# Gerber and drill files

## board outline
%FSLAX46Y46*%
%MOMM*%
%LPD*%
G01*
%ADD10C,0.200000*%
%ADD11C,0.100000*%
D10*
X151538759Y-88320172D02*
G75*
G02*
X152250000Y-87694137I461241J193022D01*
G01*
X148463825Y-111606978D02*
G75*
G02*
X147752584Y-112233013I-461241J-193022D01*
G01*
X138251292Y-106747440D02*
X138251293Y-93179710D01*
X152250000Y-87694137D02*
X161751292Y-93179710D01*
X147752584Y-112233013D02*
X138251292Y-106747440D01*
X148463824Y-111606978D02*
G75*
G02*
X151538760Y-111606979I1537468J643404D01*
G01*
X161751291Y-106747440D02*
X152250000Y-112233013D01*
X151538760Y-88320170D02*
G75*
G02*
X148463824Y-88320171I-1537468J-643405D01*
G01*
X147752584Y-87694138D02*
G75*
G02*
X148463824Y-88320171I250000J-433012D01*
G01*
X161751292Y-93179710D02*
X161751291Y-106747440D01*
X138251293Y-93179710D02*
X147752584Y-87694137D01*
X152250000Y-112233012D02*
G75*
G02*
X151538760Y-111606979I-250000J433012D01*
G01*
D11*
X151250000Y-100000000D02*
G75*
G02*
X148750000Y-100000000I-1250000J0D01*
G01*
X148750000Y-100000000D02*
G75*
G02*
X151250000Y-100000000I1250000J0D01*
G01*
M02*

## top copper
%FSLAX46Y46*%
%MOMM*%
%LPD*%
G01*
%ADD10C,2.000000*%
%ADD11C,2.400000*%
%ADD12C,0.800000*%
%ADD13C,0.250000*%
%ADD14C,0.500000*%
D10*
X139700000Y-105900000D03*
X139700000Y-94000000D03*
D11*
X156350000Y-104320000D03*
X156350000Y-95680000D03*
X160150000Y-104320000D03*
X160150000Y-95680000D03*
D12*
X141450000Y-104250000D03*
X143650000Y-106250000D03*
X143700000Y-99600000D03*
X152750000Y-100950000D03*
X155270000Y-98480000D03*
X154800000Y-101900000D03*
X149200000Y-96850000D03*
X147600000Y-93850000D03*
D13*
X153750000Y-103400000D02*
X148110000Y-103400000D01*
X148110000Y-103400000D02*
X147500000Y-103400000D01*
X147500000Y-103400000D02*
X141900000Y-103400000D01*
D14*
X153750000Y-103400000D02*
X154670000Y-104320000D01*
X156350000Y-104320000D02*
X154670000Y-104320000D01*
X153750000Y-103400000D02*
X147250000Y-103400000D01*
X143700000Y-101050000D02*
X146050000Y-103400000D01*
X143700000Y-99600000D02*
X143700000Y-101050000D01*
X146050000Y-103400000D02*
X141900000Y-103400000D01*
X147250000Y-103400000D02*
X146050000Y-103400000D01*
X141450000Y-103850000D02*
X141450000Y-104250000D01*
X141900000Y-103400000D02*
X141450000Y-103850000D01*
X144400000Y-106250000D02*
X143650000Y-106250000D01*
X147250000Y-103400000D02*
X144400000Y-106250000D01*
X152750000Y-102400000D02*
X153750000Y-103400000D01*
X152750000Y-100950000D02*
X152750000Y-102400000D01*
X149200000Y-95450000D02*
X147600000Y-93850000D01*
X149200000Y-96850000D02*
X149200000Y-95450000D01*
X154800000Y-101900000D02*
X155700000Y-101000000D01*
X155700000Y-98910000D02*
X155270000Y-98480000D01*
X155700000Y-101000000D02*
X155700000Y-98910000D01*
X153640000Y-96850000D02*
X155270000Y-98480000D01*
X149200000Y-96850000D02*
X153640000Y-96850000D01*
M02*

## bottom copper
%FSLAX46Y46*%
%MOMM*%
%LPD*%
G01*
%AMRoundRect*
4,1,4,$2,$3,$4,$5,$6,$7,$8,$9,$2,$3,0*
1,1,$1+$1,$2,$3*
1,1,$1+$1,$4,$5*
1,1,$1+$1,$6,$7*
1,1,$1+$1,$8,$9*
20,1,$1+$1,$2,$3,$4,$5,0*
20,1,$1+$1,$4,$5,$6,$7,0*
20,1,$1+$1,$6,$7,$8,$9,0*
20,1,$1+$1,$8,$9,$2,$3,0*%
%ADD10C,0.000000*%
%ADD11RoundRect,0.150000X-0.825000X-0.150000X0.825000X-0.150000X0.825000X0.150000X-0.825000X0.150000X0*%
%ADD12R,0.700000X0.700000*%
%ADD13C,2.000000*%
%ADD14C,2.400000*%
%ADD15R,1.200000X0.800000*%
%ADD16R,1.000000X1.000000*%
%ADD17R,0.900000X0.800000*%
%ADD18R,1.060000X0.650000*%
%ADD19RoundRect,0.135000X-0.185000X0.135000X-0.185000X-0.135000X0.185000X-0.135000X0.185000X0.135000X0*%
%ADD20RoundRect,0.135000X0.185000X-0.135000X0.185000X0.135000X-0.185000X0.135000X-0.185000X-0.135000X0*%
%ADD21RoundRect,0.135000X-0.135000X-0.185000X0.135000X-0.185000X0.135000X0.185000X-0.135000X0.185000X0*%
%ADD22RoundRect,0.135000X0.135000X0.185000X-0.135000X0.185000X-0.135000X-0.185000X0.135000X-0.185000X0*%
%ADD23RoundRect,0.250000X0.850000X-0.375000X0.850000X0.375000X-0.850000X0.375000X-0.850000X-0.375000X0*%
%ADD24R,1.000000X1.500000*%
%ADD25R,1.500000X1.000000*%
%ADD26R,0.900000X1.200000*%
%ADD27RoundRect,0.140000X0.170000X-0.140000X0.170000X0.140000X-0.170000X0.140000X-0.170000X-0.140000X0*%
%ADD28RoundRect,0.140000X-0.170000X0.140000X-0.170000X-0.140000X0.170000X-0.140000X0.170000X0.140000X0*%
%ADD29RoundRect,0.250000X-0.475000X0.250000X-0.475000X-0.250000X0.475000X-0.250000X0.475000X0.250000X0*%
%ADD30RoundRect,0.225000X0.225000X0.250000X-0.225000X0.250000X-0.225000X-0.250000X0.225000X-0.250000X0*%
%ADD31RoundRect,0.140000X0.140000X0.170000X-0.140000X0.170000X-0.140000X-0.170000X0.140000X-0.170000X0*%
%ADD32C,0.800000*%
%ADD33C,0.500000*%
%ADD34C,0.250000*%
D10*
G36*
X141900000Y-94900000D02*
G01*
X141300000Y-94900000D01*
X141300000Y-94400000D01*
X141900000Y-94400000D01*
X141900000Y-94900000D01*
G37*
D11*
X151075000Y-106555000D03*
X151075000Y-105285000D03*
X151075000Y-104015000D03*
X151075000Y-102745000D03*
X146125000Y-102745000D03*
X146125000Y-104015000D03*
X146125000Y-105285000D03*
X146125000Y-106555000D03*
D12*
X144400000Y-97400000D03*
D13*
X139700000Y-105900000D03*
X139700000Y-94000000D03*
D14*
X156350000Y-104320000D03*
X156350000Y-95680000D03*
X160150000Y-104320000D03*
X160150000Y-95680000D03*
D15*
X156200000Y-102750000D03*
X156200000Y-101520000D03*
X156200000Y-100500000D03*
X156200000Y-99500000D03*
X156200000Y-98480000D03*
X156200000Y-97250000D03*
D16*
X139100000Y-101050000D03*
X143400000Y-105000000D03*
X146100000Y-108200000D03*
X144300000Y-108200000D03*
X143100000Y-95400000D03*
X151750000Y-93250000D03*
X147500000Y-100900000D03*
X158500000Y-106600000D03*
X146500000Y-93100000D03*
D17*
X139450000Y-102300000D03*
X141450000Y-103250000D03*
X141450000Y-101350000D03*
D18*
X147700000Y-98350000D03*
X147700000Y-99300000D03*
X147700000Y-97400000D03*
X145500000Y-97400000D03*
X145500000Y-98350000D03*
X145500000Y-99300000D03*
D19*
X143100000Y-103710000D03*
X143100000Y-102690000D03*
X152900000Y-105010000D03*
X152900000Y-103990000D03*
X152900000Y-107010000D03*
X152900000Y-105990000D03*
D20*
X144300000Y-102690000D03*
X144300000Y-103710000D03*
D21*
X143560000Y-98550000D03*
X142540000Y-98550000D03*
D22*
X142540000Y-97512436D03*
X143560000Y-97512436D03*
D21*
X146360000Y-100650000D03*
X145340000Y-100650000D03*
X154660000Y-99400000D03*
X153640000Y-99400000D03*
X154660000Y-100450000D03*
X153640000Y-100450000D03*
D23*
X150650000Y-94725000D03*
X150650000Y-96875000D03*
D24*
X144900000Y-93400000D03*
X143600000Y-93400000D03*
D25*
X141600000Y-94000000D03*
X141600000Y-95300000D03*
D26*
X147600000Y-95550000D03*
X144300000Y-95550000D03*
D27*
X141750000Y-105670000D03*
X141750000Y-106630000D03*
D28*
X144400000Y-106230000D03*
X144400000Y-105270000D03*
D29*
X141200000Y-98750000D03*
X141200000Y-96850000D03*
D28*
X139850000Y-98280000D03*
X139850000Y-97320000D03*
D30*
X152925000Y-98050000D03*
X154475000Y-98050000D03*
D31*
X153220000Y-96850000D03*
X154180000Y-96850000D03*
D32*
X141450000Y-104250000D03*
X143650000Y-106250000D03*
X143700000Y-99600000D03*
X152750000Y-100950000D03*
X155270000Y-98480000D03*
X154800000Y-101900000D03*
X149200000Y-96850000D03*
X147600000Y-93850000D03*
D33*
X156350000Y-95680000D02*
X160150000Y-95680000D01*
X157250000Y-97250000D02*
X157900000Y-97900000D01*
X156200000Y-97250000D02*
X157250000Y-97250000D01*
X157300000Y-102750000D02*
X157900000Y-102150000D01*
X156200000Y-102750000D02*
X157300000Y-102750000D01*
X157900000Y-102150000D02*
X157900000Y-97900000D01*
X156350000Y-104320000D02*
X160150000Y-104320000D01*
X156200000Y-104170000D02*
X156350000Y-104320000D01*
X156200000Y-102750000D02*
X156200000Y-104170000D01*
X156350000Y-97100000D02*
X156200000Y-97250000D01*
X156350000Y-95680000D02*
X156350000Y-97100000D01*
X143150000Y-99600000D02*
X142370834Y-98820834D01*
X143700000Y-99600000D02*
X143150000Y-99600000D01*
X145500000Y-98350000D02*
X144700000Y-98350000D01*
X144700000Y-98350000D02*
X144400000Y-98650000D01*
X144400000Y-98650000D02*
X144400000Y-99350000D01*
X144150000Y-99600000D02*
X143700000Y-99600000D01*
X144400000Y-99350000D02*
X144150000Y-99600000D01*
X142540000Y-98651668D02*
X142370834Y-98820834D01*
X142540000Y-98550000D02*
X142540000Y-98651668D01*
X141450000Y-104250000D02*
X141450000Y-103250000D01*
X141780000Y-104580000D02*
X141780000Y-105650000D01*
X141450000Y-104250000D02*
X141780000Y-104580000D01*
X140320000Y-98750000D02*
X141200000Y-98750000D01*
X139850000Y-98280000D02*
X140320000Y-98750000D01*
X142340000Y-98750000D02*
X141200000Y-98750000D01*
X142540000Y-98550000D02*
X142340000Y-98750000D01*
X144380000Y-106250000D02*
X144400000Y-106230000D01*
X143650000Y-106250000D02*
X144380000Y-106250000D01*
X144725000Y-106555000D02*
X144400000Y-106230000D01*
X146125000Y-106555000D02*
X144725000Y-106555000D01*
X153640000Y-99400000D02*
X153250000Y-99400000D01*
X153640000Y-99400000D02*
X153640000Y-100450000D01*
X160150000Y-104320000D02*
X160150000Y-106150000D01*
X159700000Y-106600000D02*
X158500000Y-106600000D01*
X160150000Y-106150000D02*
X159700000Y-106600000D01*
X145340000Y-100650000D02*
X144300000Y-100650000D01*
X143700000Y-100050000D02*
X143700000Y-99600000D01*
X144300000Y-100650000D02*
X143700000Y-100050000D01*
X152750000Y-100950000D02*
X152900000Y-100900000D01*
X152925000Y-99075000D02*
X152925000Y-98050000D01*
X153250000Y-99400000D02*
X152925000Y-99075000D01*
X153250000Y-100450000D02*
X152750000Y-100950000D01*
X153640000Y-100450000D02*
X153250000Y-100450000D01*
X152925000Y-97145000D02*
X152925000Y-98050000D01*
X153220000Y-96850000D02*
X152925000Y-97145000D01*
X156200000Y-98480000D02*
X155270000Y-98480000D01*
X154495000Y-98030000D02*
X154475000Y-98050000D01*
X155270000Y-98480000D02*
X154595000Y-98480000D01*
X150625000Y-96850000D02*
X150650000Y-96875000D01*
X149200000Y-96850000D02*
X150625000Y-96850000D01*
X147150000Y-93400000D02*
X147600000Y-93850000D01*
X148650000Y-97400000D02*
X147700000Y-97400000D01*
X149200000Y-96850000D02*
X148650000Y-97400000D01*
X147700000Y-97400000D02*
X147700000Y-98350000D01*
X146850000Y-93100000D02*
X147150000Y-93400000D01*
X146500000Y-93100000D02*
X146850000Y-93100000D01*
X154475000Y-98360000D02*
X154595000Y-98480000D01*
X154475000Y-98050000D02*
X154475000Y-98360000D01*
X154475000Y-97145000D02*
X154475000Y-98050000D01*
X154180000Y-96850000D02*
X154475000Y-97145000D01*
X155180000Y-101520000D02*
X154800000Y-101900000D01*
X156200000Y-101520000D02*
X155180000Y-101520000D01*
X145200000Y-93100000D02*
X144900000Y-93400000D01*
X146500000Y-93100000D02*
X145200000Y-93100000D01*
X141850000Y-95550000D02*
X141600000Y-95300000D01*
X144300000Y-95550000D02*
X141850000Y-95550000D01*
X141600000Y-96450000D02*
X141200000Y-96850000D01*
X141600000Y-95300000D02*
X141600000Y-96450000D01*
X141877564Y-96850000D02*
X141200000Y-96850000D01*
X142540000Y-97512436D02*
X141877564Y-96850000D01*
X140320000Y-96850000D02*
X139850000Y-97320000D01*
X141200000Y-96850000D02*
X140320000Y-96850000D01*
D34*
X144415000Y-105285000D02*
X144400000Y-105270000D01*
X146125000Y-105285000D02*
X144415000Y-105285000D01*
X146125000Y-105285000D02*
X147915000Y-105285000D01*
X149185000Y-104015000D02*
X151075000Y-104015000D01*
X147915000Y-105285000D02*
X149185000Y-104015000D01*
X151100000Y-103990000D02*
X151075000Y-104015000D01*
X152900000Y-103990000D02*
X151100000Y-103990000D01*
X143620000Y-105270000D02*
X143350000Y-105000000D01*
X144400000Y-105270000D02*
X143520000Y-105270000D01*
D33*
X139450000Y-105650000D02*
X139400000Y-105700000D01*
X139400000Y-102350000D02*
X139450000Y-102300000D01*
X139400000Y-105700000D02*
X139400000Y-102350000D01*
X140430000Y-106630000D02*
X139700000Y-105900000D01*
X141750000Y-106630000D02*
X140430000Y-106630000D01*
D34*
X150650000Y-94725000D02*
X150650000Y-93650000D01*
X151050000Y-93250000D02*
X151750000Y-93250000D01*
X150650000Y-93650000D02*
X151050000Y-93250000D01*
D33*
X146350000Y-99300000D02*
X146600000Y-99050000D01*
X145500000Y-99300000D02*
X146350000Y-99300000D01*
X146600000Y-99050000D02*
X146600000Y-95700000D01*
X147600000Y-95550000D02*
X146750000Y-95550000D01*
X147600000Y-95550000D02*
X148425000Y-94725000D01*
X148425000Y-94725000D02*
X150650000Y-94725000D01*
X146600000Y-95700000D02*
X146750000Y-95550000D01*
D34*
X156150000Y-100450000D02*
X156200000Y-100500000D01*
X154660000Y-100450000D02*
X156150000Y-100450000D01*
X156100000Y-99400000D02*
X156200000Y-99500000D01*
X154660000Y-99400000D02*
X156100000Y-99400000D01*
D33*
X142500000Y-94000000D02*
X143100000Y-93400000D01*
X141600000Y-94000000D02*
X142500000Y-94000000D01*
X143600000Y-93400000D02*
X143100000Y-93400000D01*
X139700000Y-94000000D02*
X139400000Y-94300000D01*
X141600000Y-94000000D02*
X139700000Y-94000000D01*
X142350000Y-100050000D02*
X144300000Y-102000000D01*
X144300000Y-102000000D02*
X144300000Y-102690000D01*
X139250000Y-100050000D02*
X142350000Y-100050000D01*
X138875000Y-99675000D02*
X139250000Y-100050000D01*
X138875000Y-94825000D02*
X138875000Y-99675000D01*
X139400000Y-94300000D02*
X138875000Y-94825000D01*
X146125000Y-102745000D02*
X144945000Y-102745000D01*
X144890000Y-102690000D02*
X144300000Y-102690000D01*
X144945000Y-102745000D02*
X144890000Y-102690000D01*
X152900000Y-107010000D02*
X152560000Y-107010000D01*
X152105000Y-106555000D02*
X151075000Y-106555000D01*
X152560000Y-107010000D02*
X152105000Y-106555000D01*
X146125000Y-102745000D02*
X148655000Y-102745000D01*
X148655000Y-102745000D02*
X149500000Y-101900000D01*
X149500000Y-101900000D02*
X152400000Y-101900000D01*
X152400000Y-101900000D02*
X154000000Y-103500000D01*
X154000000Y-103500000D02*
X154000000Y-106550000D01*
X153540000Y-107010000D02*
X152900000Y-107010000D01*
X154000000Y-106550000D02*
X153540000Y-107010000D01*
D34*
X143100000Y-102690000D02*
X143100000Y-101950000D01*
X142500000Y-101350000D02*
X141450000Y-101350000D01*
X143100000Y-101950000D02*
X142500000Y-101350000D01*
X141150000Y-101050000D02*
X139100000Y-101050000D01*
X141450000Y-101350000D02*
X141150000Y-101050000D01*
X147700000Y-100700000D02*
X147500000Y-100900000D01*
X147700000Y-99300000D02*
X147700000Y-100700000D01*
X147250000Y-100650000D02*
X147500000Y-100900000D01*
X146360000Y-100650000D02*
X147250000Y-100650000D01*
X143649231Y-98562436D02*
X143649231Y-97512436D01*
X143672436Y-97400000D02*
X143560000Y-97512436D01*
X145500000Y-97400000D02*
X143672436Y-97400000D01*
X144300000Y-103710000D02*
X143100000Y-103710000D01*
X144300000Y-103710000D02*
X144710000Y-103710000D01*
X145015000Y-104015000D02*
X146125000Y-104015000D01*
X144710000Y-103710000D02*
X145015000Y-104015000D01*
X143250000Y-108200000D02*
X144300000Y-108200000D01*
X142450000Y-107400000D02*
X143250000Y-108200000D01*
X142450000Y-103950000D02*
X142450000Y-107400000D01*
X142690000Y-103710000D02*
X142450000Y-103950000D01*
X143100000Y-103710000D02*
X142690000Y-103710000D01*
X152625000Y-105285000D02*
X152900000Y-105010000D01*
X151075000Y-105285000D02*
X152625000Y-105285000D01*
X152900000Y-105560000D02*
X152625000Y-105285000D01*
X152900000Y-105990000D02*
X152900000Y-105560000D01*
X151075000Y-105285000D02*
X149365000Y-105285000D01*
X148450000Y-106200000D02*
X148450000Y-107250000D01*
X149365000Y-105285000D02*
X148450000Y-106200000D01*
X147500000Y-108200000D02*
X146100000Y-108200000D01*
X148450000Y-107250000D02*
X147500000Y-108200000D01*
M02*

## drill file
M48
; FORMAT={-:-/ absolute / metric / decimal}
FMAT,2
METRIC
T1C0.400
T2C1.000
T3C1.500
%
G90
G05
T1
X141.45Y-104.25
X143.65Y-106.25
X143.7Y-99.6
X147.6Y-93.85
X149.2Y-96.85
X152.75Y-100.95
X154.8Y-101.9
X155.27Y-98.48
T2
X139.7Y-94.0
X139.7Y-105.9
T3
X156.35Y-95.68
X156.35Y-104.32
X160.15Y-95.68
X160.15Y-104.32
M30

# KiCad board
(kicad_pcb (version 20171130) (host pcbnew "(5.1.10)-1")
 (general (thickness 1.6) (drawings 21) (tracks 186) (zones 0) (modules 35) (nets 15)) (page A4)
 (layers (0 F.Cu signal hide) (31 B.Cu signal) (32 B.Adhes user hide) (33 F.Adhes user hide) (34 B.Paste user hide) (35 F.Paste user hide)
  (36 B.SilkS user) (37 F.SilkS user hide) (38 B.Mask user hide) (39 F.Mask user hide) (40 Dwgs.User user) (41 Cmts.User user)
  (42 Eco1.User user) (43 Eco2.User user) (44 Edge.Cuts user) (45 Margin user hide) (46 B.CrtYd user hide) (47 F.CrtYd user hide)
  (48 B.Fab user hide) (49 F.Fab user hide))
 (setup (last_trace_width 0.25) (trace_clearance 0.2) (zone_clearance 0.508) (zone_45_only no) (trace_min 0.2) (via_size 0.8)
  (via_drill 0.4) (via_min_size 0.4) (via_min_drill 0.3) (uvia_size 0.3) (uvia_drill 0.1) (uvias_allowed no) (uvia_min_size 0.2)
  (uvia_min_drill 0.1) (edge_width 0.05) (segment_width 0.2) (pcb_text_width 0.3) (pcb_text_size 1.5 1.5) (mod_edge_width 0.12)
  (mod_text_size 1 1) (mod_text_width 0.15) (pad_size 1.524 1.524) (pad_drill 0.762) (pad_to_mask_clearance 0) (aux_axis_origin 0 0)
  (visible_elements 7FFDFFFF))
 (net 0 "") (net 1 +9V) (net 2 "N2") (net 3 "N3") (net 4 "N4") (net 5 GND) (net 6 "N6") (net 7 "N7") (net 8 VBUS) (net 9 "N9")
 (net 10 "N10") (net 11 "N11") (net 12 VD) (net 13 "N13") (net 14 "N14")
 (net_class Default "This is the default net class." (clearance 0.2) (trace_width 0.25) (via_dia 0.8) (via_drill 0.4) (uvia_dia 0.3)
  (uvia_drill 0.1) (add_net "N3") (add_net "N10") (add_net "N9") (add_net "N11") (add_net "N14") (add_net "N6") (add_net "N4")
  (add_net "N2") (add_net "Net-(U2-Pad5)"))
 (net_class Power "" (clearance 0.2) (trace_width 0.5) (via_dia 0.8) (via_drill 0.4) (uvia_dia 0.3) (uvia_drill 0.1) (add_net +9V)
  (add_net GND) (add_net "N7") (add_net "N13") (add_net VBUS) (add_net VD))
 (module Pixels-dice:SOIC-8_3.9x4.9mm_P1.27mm (layer B.Cu) (at 148.6 104.65 90)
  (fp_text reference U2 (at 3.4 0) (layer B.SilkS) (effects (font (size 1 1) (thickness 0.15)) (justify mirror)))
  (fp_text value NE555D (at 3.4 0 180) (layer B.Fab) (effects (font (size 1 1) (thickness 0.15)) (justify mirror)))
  (pad 8 smd roundrect (at -1.905 2.475) (size 1.95 0.6) (layers B.Cu B.Paste B.Mask) (roundrect_rratio 0.25) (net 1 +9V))
  (pad 7 smd roundrect (at -0.635 2.475) (size 1.95 0.6) (layers B.Cu B.Paste B.Mask) (roundrect_rratio 0.25) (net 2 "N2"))
  (pad 6 smd roundrect (at 0.635 2.475) (size 1.95 0.6) (layers B.Cu B.Paste B.Mask) (roundrect_rratio 0.25) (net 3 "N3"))
  (pad 5 smd roundrect (at 1.905 2.475) (size 1.95 0.6) (layers B.Cu B.Paste B.Mask) (roundrect_rratio 0.25))
  (pad 4 smd roundrect (at 1.905 -2.475) (size 1.95 0.6) (layers B.Cu B.Paste B.Mask) (roundrect_rratio 0.25) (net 1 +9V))
  (pad 3 smd roundrect (at 0.635 -2.475) (size 1.95 0.6) (layers B.Cu B.Paste B.Mask) (roundrect_rratio 0.25) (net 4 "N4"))
  (pad 2 smd roundrect (at -0.635 -2.475) (size 1.95 0.6) (layers B.Cu B.Paste B.Mask) (roundrect_rratio 0.25) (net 3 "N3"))
  (pad 1 smd roundrect (at -1.905 -2.475) (size 1.95 0.6) (layers B.Cu B.Paste B.Mask) (roundrect_rratio 0.25) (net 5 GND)))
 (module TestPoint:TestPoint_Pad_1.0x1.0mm (layer B.Cu) (at 144.4 97.4)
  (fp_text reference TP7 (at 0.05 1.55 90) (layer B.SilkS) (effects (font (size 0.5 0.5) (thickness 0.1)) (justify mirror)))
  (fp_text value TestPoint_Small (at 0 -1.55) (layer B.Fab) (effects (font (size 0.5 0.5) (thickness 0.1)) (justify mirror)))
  (pad 1 smd rect (at 0 0) (size 0.7 0.7) (layers B.Cu B.Mask) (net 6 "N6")))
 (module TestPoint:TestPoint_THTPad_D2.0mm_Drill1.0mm (layer F.Cu) (at 139.7 105.9)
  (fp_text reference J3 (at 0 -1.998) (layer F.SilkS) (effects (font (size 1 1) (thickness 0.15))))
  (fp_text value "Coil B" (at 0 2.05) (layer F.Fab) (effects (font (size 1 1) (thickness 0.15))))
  (pad 1 thru_hole circle (at 0 0) (size 2 2) (drill 1) (layers *.Cu *.Mask) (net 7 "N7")))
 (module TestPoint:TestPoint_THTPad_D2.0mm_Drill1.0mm (layer F.Cu) (at 139.7 94)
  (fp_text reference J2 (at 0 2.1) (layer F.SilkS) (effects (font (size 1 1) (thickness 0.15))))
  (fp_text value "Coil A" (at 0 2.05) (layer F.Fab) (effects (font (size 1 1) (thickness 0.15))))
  (pad 1 thru_hole circle (at 0 0) (size 2 2) (drill 1) (layers *.Cu *.Mask) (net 1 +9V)))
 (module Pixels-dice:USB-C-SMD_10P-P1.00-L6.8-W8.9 (layer B.Cu) (at 158.35 100)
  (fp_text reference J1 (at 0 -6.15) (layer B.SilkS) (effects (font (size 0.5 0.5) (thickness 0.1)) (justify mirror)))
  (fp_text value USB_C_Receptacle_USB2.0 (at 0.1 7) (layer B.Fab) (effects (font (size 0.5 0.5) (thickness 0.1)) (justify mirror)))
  (pad S1 thru_hole circle (at -2 4.32 270) (size 2.4 2.4) (drill 1.5) (layers *.Cu *.Mask) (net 5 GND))
  (pad S1 thru_hole circle (at -2 -4.32 270) (size 2.4 2.4) (drill 1.5) (layers *.Cu *.Mask) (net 5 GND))
  (pad S1 thru_hole circle (at 1.8 4.32 270) (size 2.4 2.4) (drill 1.5) (layers *.Cu *.Mask) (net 5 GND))
  (pad S1 thru_hole circle (at 1.8 -4.32 270) (size 2.4 2.4) (drill 1.5) (layers *.Cu *.Mask) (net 5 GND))
  (pad A12 smd rect (at -2.15 2.75 270) (size 0.8 1.2) (layers B.Cu B.Paste B.Mask) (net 5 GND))
  (pad A9 smd rect (at -2.15 1.52 270) (size 0.8 1.2) (layers B.Cu B.Paste B.Mask) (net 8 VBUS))
  (pad B5 smd rect (at -2.15 0.5 270) (size 0.8 1.2) (layers B.Cu B.Paste B.Mask) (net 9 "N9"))
  (pad A5 smd rect (at -2.15 -0.5 270) (size 0.8 1.2) (layers B.Cu B.Paste B.Mask) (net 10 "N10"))
  (pad B9 smd rect (at -2.15 -1.52 270) (size 0.8 1.2) (layers B.Cu B.Paste B.Mask) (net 8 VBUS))
  (pad B12 smd rect (at -2.15 -2.75 270) (size 0.8 1.2) (layers B.Cu B.Paste B.Mask) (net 5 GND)))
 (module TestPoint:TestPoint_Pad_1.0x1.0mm (layer B.Cu) (at 139.1 101.05)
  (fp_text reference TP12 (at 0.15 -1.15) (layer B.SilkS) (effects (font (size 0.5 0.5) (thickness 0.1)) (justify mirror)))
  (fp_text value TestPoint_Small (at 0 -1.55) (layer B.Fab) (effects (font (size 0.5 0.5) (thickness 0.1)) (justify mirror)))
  (pad 1 smd rect (at 0 0) (size 1 1) (layers B.Cu B.Mask) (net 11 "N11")))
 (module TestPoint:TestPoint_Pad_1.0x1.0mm (layer B.Cu) (at 143.4 105)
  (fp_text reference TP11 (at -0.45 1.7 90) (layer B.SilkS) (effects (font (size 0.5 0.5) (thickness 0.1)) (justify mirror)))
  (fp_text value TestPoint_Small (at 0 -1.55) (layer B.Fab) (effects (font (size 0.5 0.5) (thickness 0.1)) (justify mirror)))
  (pad 1 smd rect (at 0 0) (size 1 1) (layers B.Cu B.Mask) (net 3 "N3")))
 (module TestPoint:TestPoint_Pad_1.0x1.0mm (layer B.Cu) (at 146.1 108.2)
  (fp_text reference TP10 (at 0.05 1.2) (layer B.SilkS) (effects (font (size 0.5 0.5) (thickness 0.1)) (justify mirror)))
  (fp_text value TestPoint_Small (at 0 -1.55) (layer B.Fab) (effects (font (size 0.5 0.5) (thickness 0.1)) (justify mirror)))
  (pad 1 smd rect (at 0 0) (size 1 1) (layers B.Cu B.Mask) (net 2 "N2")))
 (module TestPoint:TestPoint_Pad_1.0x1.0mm (layer B.Cu) (at 144.3 108.2)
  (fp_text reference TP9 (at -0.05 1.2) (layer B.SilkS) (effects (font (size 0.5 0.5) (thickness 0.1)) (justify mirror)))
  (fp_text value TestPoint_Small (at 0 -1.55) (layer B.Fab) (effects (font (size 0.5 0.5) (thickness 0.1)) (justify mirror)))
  (pad 1 smd rect (at 0 0) (size 1 1) (layers B.Cu B.Mask) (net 4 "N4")))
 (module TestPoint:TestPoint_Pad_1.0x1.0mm (layer B.Cu) (at 143.1 95.4)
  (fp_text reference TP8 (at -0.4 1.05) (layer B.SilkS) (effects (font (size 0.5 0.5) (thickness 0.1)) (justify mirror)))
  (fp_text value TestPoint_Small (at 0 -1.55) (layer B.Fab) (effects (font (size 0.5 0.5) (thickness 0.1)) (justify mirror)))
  (pad 1 smd rect (at 0 0) (size 1 1) (layers B.Cu B.Mask) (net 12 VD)))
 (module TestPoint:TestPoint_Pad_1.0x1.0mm (layer B.Cu) (at 151.75 93.25)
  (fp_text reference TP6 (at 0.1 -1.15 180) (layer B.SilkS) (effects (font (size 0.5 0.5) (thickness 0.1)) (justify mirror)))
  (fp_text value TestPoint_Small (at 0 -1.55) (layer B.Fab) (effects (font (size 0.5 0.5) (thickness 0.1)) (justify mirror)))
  (pad 1 smd rect (at 0 0) (size 1 1) (layers B.Cu B.Mask) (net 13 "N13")))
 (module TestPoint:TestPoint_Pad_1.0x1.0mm (layer B.Cu) (at 147.5 100.9)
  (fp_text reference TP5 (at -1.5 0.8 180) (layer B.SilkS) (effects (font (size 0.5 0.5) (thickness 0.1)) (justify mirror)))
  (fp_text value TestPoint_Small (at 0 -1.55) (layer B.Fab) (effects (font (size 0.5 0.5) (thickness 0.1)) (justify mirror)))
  (pad 1 smd rect (at 0 0) (size 1 1) (layers B.Cu B.Mask) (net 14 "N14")))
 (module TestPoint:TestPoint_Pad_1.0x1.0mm (layer B.Cu) (at 158.5 106.6)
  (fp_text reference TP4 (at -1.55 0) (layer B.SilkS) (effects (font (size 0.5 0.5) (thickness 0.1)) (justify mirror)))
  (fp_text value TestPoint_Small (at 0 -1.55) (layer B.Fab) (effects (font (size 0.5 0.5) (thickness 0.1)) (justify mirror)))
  (pad 1 smd rect (at 0 0) (size 1 1) (layers B.Cu B.Mask) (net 5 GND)))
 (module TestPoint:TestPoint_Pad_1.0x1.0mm (layer B.Cu) (at 146.5 93.1)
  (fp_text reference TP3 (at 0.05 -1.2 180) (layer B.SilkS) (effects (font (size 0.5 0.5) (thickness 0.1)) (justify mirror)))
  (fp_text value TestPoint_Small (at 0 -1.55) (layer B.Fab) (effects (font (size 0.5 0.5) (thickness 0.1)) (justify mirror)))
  (pad 1 smd rect (at 0 0) (size 1 1) (layers B.Cu B.Mask) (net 8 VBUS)))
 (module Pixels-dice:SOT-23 (layer B.Cu) (at 140.45 102.3)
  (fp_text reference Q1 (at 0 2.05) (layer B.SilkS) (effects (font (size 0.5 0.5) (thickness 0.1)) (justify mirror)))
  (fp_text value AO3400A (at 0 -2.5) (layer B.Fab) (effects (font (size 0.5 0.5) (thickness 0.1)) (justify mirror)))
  (pad 3 smd rect (at -1 0 180) (size 0.9 0.8) (layers B.Cu B.Paste B.Mask) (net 7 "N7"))
  (pad 2 smd rect (at 1 0.95 180) (size 0.9 0.8) (layers B.Cu B.Paste B.Mask) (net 5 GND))
  (pad 1 smd rect (at 1 -0.95 180) (size 0.9 0.8) (layers B.Cu B.Paste B.Mask) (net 11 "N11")))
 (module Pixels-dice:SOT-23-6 (layer B.Cu) (at 146.6 98.35 180)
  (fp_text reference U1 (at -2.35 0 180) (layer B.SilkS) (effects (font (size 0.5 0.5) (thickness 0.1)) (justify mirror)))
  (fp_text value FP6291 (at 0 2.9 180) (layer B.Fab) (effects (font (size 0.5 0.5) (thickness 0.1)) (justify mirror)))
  (pad 5 smd rect (at -1.1 0) (size 1.06 0.65) (layers B.Cu B.Paste B.Mask) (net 8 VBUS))
  (pad 6 smd rect (at -1.1 -0.95) (size 1.06 0.65) (layers B.Cu B.Paste B.Mask) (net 14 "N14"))
  (pad 4 smd rect (at -1.1 0.95) (size 1.06 0.65) (layers B.Cu B.Paste B.Mask) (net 8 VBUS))
  (pad 3 smd rect (at 1.1 0.95) (size 1.06 0.65) (layers B.Cu B.Paste B.Mask) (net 6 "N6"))
  (pad 2 smd rect (at 1.1 0) (size 1.06 0.65) (layers B.Cu B.Paste B.Mask) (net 5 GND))
  (pad 1 smd rect (at 1.1 -0.95) (size 1.06 0.65) (layers B.Cu B.Paste B.Mask) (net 13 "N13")))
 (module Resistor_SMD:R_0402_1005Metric (layer B.Cu) (at 143.1 103.2 270)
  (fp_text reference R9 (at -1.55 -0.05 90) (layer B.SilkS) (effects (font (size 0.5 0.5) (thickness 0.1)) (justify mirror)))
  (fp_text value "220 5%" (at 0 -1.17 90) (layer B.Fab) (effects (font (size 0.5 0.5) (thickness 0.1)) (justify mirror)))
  (pad 2 smd roundrect (at 0.51 0 270) (size 0.54 0.64) (layers B.Cu B.Paste B.Mask) (roundrect_rratio 0.25) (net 4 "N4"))
  (pad 1 smd roundrect (at -0.51 0 270) (size 0.54 0.64) (layers B.Cu B.Paste B.Mask) (roundrect_rratio 0.25) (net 11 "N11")))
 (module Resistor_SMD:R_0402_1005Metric (layer B.Cu) (at 152.9 104.5 270)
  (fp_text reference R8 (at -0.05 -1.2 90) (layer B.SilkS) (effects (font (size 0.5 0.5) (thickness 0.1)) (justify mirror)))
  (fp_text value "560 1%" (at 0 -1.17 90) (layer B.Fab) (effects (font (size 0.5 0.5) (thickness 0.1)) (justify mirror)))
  (pad 2 smd roundrect (at 0.51 0 270) (size 0.54 0.64) (layers B.Cu B.Paste B.Mask) (roundrect_rratio 0.25) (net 2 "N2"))
  (pad 1 smd roundrect (at -0.51 0 270) (size 0.54 0.64) (layers B.Cu B.Paste B.Mask) (roundrect_rratio 0.25) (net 3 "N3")))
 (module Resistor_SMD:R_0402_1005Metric (layer B.Cu) (at 152.9 106.5 270)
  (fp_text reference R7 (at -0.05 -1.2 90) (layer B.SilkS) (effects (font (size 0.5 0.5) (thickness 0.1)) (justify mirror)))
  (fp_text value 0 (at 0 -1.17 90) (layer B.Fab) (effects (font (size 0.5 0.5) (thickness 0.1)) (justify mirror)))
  (pad 2 smd roundrect (at 0.51 0 270) (size 0.54 0.64) (layers B.Cu B.Paste B.Mask) (roundrect_rratio 0.25) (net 1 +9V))
  (pad 1 smd roundrect (at -0.51 0 270) (size 0.54 0.64) (layers B.Cu B.Paste B.Mask) (roundrect_rratio 0.25) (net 2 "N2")))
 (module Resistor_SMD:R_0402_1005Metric (layer B.Cu) (at 144.3 103.2 90)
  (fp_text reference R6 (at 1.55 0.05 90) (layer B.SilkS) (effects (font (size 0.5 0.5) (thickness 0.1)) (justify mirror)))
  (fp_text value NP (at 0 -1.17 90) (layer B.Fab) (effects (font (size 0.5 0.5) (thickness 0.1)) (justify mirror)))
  (pad 2 smd roundrect (at 0.51 0 90) (size 0.54 0.64) (layers B.Cu B.Paste B.Mask) (roundrect_rratio 0.25) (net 1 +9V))
  (pad 1 smd roundrect (at -0.51 0 90) (size 0.54 0.64) (layers B.Cu B.Paste B.Mask) (roundrect_rratio 0.25) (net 4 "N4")))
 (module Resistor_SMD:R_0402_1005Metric (layer B.Cu) (at 143.05 98.55)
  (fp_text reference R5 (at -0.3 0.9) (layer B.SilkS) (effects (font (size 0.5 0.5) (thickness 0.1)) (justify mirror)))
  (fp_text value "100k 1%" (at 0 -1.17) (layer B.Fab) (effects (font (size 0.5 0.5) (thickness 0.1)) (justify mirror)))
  (pad 2 smd roundrect (at 0.51 0) (size 0.54 0.64) (layers B.Cu B.Paste B.Mask) (roundrect_rratio 0.25) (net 6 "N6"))
  (pad 1 smd roundrect (at -0.51 0) (size 0.54 0.64) (layers B.Cu B.Paste B.Mask) (roundrect_rratio 0.25) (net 5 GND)))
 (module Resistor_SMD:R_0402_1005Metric (layer B.Cu) (at 143.05 97.512436 180)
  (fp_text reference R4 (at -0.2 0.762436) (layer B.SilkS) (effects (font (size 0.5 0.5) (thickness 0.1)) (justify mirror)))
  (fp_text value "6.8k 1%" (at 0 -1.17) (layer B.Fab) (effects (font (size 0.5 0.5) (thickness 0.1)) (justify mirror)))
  (pad 2 smd roundrect (at 0.51 0 180) (size 0.54 0.64) (layers B.Cu B.Paste B.Mask) (roundrect_rratio 0.25) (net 12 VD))
  (pad 1 smd roundrect (at -0.51 0 180) (size 0.54 0.64) (layers B.Cu B.Paste B.Mask) (roundrect_rratio 0.25) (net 6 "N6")))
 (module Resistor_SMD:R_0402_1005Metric (layer B.Cu) (at 145.85 100.65)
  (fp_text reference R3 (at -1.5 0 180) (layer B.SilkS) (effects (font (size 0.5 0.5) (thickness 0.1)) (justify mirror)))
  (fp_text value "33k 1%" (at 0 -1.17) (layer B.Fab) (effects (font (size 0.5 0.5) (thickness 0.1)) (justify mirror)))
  (pad 2 smd roundrect (at 0.51 0) (size 0.54 0.64) (layers B.Cu B.Paste B.Mask) (roundrect_rratio 0.25) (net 14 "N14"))
  (pad 1 smd roundrect (at -0.51 0) (size 0.54 0.64) (layers B.Cu B.Paste B.Mask) (roundrect_rratio 0.25) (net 5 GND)))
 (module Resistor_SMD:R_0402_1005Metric (layer B.Cu) (at 154.15 99.4)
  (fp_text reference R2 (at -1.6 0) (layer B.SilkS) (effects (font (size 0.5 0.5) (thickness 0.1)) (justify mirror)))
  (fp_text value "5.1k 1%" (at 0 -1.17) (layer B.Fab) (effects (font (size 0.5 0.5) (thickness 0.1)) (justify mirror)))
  (pad 2 smd roundrect (at 0.51 0) (size 0.54 0.64) (layers B.Cu B.Paste B.Mask) (roundrect_rratio 0.25) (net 10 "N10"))
  (pad 1 smd roundrect (at -0.51 0) (size 0.54 0.64) (layers B.Cu B.Paste B.Mask) (roundrect_rratio 0.25) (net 5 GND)))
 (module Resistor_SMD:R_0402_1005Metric (layer B.Cu) (at 154.15 100.45)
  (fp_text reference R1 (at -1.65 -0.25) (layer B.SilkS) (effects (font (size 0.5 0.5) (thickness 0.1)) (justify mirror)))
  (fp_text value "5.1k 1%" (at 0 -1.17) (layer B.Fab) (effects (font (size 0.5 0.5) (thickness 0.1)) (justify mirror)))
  (pad 2 smd roundrect (at 0.51 0) (size 0.54 0.64) (layers B.Cu B.Paste B.Mask) (roundrect_rratio 0.25) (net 9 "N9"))
  (pad 1 smd roundrect (at -0.51 0) (size 0.54 0.64) (layers B.Cu B.Paste B.Mask) (roundrect_rratio 0.25) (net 5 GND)))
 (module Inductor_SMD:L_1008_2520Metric (layer B.Cu) (at 150.65 95.8 90)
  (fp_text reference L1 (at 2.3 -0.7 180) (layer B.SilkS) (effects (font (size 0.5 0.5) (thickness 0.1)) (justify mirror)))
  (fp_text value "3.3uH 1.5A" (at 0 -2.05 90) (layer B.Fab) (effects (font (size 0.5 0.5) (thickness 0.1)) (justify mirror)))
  (pad 2 smd roundrect (at 1.075 0 90) (size 1.25 2.2) (layers B.Cu B.Paste B.Mask) (roundrect_rratio 0.2) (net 13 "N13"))
  (pad 1 smd roundrect (at -1.075 0 90) (size 1.25 2.2) (layers B.Cu B.Paste B.Mask) (roundrect_rratio 0.2) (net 8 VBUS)))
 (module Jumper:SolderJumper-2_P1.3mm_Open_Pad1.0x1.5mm (layer B.Cu) (at 144.25 93.4 180)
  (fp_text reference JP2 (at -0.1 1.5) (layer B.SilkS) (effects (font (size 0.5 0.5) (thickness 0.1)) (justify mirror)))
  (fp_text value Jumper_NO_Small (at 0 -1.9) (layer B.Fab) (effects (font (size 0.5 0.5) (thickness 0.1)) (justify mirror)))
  (pad 1 smd rect (at -0.65 0 180) (size 1 1.5) (layers B.Cu B.Mask) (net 8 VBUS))
  (pad 2 smd rect (at 0.65 0 180) (size 1 1.5) (layers B.Cu B.Mask) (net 1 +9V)))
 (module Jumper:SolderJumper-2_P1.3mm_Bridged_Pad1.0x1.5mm (layer B.Cu) (at 141.6 94.65 90)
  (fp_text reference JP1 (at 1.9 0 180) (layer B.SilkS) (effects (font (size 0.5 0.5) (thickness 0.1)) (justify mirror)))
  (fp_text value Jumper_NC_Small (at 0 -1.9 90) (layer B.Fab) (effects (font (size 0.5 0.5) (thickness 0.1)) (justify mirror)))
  (fp_poly (pts (xy -0.25 0.3) (xy 0.25 0.3) (xy 0.25 -0.3) (xy -0.25 -0.3)) (layer B.Cu) (width 0))
  (pad 2 smd rect (at 0.65 0 90) (size 1 1.5) (layers B.Cu B.Mask) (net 1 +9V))
  (pad 1 smd rect (at -0.65 0 90) (size 1 1.5) (layers B.Cu B.Mask) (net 12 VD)))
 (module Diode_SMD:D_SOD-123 (layer B.Cu) (at 145.95 95.55)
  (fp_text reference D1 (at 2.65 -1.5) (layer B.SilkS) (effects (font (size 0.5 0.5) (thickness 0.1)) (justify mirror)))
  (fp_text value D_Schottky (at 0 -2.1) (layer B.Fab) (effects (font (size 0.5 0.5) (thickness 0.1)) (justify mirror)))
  (pad 2 smd rect (at 1.65 0) (size 0.9 1.2) (layers B.Cu B.Paste B.Mask) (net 13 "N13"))
  (pad 1 smd rect (at -1.65 0) (size 0.9 1.2) (layers B.Cu B.Paste B.Mask) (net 12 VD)))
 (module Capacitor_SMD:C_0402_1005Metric (layer B.Cu) (at 141.75 106.15 90)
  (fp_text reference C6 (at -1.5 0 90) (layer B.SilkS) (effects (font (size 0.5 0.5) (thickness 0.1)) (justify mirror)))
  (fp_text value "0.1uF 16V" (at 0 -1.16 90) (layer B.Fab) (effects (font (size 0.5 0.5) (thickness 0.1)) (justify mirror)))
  (pad 2 smd roundrect (at 0.48 0 90) (size 0.56 0.62) (layers B.Cu B.Paste B.Mask) (roundrect_rratio 0.25) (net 5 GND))
  (pad 1 smd roundrect (at -0.48 0 90) (size 0.56 0.62) (layers B.Cu B.Paste B.Mask) (roundrect_rratio 0.25) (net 7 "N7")))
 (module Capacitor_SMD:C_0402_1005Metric (layer B.Cu) (at 144.4 105.75 270)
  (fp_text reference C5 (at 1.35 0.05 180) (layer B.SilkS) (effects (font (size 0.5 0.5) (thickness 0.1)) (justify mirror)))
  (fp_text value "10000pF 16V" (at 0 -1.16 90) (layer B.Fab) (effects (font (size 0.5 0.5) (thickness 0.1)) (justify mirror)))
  (pad 2 smd roundrect (at 0.48 0 270) (size 0.56 0.62) (layers B.Cu B.Paste B.Mask) (roundrect_rratio 0.25) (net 5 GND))
  (pad 1 smd roundrect (at -0.48 0 270) (size 0.56 0.62) (layers B.Cu B.Paste B.Mask) (roundrect_rratio 0.25) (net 3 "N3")))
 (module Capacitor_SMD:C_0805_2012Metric (layer B.Cu) (at 141.2 97.8 270)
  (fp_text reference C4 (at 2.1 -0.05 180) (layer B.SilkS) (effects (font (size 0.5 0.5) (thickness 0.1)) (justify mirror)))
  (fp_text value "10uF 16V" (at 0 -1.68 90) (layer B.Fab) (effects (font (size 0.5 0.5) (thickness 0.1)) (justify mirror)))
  (pad 2 smd roundrect (at 0.95 0 270) (size 1 1.45) (layers B.Cu B.Paste B.Mask) (roundrect_rratio 0.25) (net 5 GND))
  (pad 1 smd roundrect (at -0.95 0 270) (size 1 1.45) (layers B.Cu B.Paste B.Mask) (roundrect_rratio 0.25) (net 12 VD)))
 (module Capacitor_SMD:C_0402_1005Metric (layer B.Cu) (at 139.85 97.8 270)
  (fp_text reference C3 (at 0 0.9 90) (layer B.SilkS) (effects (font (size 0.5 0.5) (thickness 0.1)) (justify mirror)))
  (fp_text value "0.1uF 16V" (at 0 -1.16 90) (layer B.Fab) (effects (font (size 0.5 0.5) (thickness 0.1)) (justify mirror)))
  (pad 2 smd roundrect (at 0.48 0 270) (size 0.56 0.62) (layers B.Cu B.Paste B.Mask) (roundrect_rratio 0.25) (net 5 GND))
  (pad 1 smd roundrect (at -0.48 0 270) (size 0.56 0.62) (layers B.Cu B.Paste B.Mask) (roundrect_rratio 0.25) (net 12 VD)))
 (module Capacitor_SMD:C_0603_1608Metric (layer B.Cu) (at 153.7 98.05 180)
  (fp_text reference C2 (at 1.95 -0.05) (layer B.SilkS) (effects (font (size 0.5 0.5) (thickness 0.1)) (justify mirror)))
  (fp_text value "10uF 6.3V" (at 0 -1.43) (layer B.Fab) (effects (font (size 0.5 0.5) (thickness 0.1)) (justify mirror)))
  (pad 2 smd roundrect (at 0.775 0 180) (size 0.9 0.95) (layers B.Cu B.Paste B.Mask) (roundrect_rratio 0.25) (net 5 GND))
  (pad 1 smd roundrect (at -0.775 0 180) (size 0.9 0.95) (layers B.Cu B.Paste B.Mask) (roundrect_rratio 0.25) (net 8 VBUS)))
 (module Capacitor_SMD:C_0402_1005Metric (layer B.Cu) (at 153.7 96.85 180)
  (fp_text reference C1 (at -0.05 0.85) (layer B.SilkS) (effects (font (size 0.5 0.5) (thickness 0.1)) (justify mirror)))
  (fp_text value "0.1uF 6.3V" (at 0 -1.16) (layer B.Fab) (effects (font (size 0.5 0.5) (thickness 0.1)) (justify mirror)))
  (pad 2 smd roundrect (at 0.48 0 180) (size 0.56 0.62) (layers B.Cu B.Paste B.Mask) (roundrect_rratio 0.25) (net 5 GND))
  (pad 1 smd roundrect (at -0.48 0 180) (size 0.56 0.62) (layers B.Cu B.Paste B.Mask) (roundrect_rratio 0.25) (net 8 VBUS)))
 (gr_arc (start 152 88.12715) (end 152.25 87.694137) (angle -142.7084941) (layer Edge.Cuts) (width 0.2))
 (gr_arc (start 148.002584 111.8) (end 147.752584 112.233013) (angle -142.7084941) (layer Edge.Cuts) (width 0.2))
 (gr_line (start 138.251292 106.74744) (end 138.251293 93.17971) (layer Edge.Cuts) (width 0.2))
 (gr_line (start 152.25 87.694137) (end 161.751292 93.17971) (layer Edge.Cuts) (width 0.2))
 (gr_line (start 147.752584 112.233013) (end 138.251292 106.74744) (layer Edge.Cuts) (width 0.2))
 (gr_arc (start 150.001292 110.963574) (end 151.53876 111.606979) (angle -225.4169678) (layer Edge.Cuts) (width 0.2))
 (gr_line (start 161.751291 106.74744) (end 152.25 112.233013) (layer Edge.Cuts) (width 0.2))
 (gr_arc (start 150.001292 88.963575) (end 148.463824 88.320171) (angle -225.4169678) (layer Edge.Cuts) (width 0.2))
 (gr_arc (start 148.002584 88.12715) (end 148.463824 88.320171) (angle -142.7084738) (layer Edge.Cuts) (width 0.2))
 (gr_line (start 161.751292 93.17971) (end 161.751291 106.74744) (layer Edge.Cuts) (width 0.2))
 (gr_line (start 138.251293 93.17971) (end 147.752584 87.694137) (layer Edge.Cuts) (width 0.2))
 (gr_arc (start 152 111.8) (end 151.53876 111.606979) (angle -142.7084738) (layer Edge.Cuts) (width 0.2))
 (gr_circle (center 150 100) (end 151.25 100) (layer Edge.Cuts) (width 0.1))
 (via (at 141.45 104.25) (size 0.8) (drill 0.4) (layers F.Cu B.Cu) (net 5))
 (via (at 143.65 106.25) (size 0.8) (drill 0.4) (layers F.Cu B.Cu) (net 5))
 (via (at 143.7 99.6) (size 0.8) (drill 0.4) (layers F.Cu B.Cu) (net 5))
 (segment (start 153.75 103.4) (end 148.11 103.4) (width 0.25) (layer F.Cu) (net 5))
 (segment (start 148.11 103.4) (end 147.5 103.4) (width 0.25) (layer F.Cu) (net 5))
 (segment (start 147.5 103.4) (end 141.9 103.4) (width 0.25) (layer F.Cu) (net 5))
 (segment (start 153.75 103.4) (end 154.67 104.32) (width 0.5) (layer F.Cu) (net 5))
 (segment (start 156.35 104.32) (end 154.67 104.32) (width 0.5) (layer F.Cu) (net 5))
 (segment (start 153.75 103.4) (end 147.25 103.4) (width 0.5) (layer F.Cu) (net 5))
 (segment (start 143.7 101.05) (end 146.05 103.4) (width 0.5) (layer F.Cu) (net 5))
 (segment (start 143.7 99.6) (end 143.7 101.05) (width 0.5) (layer F.Cu) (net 5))
 (segment (start 146.05 103.4) (end 141.9 103.4) (width 0.5) (layer F.Cu) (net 5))
 (segment (start 147.25 103.4) (end 146.05 103.4) (width 0.5) (layer F.Cu) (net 5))
 (segment (start 156.35 95.68) (end 160.15 95.68) (width 0.5) (layer B.Cu) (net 5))
 (segment (start 157.25 97.25) (end 157.9 97.9) (width 0.5) (layer B.Cu) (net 5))
 (segment (start 156.2 97.25) (end 157.25 97.25) (width 0.5) (layer B.Cu) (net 5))
 (segment (start 157.3 102.75) (end 157.9 102.15) (width 0.5) (layer B.Cu) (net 5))
 (segment (start 156.2 102.75) (end 157.3 102.75) (width 0.5) (layer B.Cu) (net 5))
 (segment (start 157.9 102.15) (end 157.9 97.9) (width 0.5) (layer B.Cu) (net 5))
 (segment (start 156.35 104.32) (end 160.15 104.32) (width 0.5) (layer B.Cu) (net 5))
 (segment (start 156.2 104.17) (end 156.35 104.32) (width 0.5) (layer B.Cu) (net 5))
 (segment (start 156.2 102.75) (end 156.2 104.17) (width 0.5) (layer B.Cu) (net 5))
 (segment (start 156.35 97.1) (end 156.2 97.25) (width 0.5) (layer B.Cu) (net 5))
 (segment (start 156.35 95.68) (end 156.35 97.1) (width 0.5) (layer B.Cu) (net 5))
 (segment (start 143.15 99.6) (end 142.370834 98.820834) (width 0.5) (layer B.Cu) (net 5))
 (segment (start 143.7 99.6) (end 143.15 99.6) (width 0.5) (layer B.Cu) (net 5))
 (segment (start 145.5 98.35) (end 144.7 98.35) (width 0.5) (layer B.Cu) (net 5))
 (segment (start 144.7 98.35) (end 144.4 98.65) (width 0.5) (layer B.Cu) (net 5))
 (segment (start 144.4 98.65) (end 144.4 99.35) (width 0.5) (layer B.Cu) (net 5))
 (segment (start 144.15 99.6) (end 143.7 99.6) (width 0.5) (layer B.Cu) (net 5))
 (segment (start 144.4 99.35) (end 144.15 99.6) (width 0.5) (layer B.Cu) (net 5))
 (segment (start 142.54 98.651668) (end 142.370834 98.820834) (width 0.5) (layer B.Cu) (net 5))
 (segment (start 142.54 98.55) (end 142.54 98.651668) (width 0.5) (layer B.Cu) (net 5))
 (segment (start 141.45 104.25) (end 141.45 103.25) (width 0.5) (layer B.Cu) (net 5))
 (segment (start 141.78 104.58) (end 141.78 105.65) (width 0.5) (layer B.Cu) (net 5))
 (segment (start 141.45 104.25) (end 141.78 104.58) (width 0.5) (layer B.Cu) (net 5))
 (segment (start 141.45 103.85) (end 141.45 104.25) (width 0.5) (layer F.Cu) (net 5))
 (segment (start 141.9 103.4) (end 141.45 103.85) (width 0.5) (layer F.Cu) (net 5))
 (segment (start 140.32 98.75) (end 141.2 98.75) (width 0.5) (layer B.Cu) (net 5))
 (segment (start 139.85 98.28) (end 140.32 98.75) (width 0.5) (layer B.Cu) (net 5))
 (segment (start 142.34 98.75) (end 141.2 98.75) (width 0.5) (layer B.Cu) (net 5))
 (segment (start 142.54 98.55) (end 142.34 98.75) (width 0.5) (layer B.Cu) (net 5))
 (segment (start 144.38 106.25) (end 144.4 106.23) (width 0.5) (layer B.Cu) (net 5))
 (segment (start 143.65 106.25) (end 144.38 106.25) (width 0.5) (layer B.Cu) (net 5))
 (segment (start 144.725 106.555) (end 144.4 106.23) (width 0.5) (layer B.Cu) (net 5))
 (segment (start 146.125 106.555) (end 144.725 106.555) (width 0.5) (layer B.Cu) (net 5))
 (segment (start 144.4 106.25) (end 143.65 106.25) (width 0.5) (layer F.Cu) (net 5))
 (segment (start 147.25 103.4) (end 144.4 106.25) (width 0.5) (layer F.Cu) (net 5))
 (segment (start 153.64 99.4) (end 153.25 99.4) (width 0.5) (layer B.Cu) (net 5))
 (segment (start 153.64 99.4) (end 153.64 100.45) (width 0.5) (layer B.Cu) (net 5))
 (segment (start 160.15 104.32) (end 160.15 106.15) (width 0.5) (layer B.Cu) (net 5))
 (segment (start 159.7 106.6) (end 158.5 106.6) (width 0.5) (layer B.Cu) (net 5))
 (segment (start 160.15 106.15) (end 159.7 106.6) (width 0.5) (layer B.Cu) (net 5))
 (segment (start 145.34 100.65) (end 144.3 100.65) (width 0.5) (layer B.Cu) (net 5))
 (segment (start 143.7 100.05) (end 143.7 99.6) (width 0.5) (layer B.Cu) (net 5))
 (segment (start 144.3 100.65) (end 143.7 100.05) (width 0.5) (layer B.Cu) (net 5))
 (via (at 152.75 100.95) (size 0.8) (drill 0.4) (layers F.Cu B.Cu) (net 5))
 (segment (start 152.75 100.95) (end 152.9 100.9) (width 0.5) (layer B.Cu) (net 5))
 (segment (start 152.75 102.4) (end 153.75 103.4) (width 0.5) (layer F.Cu) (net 5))
 (segment (start 152.75 100.95) (end 152.75 102.4) (width 0.5) (layer F.Cu) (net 5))
 (segment (start 152.925 99.075) (end 152.925 98.05) (width 0.5) (layer B.Cu) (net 5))
 (segment (start 153.25 99.4) (end 152.925 99.075) (width 0.5) (layer B.Cu) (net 5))
 (segment (start 153.25 100.45) (end 152.75 100.95) (width 0.5) (layer B.Cu) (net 5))
 (segment (start 153.64 100.45) (end 153.25 100.45) (width 0.5) (layer B.Cu) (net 5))
 (segment (start 152.925 97.145) (end 152.925 98.05) (width 0.5) (layer B.Cu) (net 5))
 (segment (start 153.22 96.85) (end 152.925 97.145) (width 0.5) (layer B.Cu) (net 5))
 (via (at 155.27 98.48) (size 0.8) (drill 0.4) (layers F.Cu B.Cu) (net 8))
 (via (at 154.8 101.9) (size 0.8) (drill 0.4) (layers F.Cu B.Cu) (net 8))
 (via (at 149.2 96.85) (size 0.8) (drill 0.4) (layers F.Cu B.Cu) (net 8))
 (via (at 147.6 93.85) (size 0.8) (drill 0.4) (layers F.Cu B.Cu) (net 8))
 (segment (start 149.2 95.45) (end 147.6 93.85) (width 0.5) (layer F.Cu) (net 8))
 (segment (start 149.2 96.85) (end 149.2 95.45) (width 0.5) (layer F.Cu) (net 8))
 (segment (start 156.2 98.48) (end 155.27 98.48) (width 0.5) (layer B.Cu) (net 8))
 (segment (start 154.495 98.03) (end 154.475 98.05) (width 0.5) (layer B.Cu) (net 8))
 (segment (start 155.27 98.48) (end 154.595 98.48) (width 0.5) (layer B.Cu) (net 8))
 (segment (start 150.625 96.85) (end 150.65 96.875) (width 0.5) (layer B.Cu) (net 8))
 (segment (start 149.2 96.85) (end 150.625 96.85) (width 0.5) (layer B.Cu) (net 8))
 (segment (start 147.15 93.4) (end 147.6 93.85) (width 0.5) (layer B.Cu) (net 8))
 (segment (start 148.65 97.4) (end 147.7 97.4) (width 0.5) (layer B.Cu) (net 8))
 (segment (start 149.2 96.85) (end 148.65 97.4) (width 0.5) (layer B.Cu) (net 8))
 (segment (start 147.7 97.4) (end 147.7 98.35) (width 0.5) (layer B.Cu) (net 8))
 (segment (start 146.85 93.1) (end 147.15 93.4) (width 0.5) (layer B.Cu) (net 8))
 (segment (start 146.5 93.1) (end 146.85 93.1) (width 0.5) (layer B.Cu) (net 8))
 (segment (start 154.8 101.9) (end 155.7 101) (width 0.5) (layer F.Cu) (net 8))
 (segment (start 155.7 98.91) (end 155.27 98.48) (width 0.5) (layer F.Cu) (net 8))
 (segment (start 155.7 101) (end 155.7 98.91) (width 0.5) (layer F.Cu) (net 8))
 (segment (start 153.64 96.85) (end 155.27 98.48) (width 0.5) (layer F.Cu) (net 8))
 (segment (start 149.2 96.85) (end 153.64 96.85) (width 0.5) (layer F.Cu) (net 8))
 (segment (start 154.475 98.36) (end 154.595 98.48) (width 0.5) (layer B.Cu) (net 8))
 (segment (start 154.475 98.05) (end 154.475 98.36) (width 0.5) (layer B.Cu) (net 8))
 (segment (start 154.475 97.145) (end 154.475 98.05) (width 0.5) (layer B.Cu) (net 8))
 (segment (start 154.18 96.85) (end 154.475 97.145) (width 0.5) (layer B.Cu) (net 8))
 (segment (start 155.18 101.52) (end 154.8 101.9) (width 0.5) (layer B.Cu) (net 8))
 (segment (start 156.2 101.52) (end 155.18 101.52) (width 0.5) (layer B.Cu) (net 8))
 (segment (start 145.2 93.1) (end 144.9 93.4) (width 0.5) (layer B.Cu) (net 8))
 (segment (start 146.5 93.1) (end 145.2 93.1) (width 0.5) (layer B.Cu) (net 8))
 (segment (start 141.85 95.55) (end 141.6 95.3) (width 0.5) (layer B.Cu) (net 12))
 (segment (start 144.3 95.55) (end 141.85 95.55) (width 0.5) (layer B.Cu) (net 12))
 (segment (start 141.6 96.45) (end 141.2 96.85) (width 0.5) (layer B.Cu) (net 12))
 (segment (start 141.6 95.3) (end 141.6 96.45) (width 0.5) (layer B.Cu) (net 12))
 (segment (start 141.877564 96.85) (end 141.2 96.85) (width 0.5) (layer B.Cu) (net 12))
 (segment (start 142.54 97.512436) (end 141.877564 96.85) (width 0.5) (layer B.Cu) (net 12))
 (segment (start 140.32 96.85) (end 139.85 97.32) (width 0.5) (layer B.Cu) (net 12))
 (segment (start 141.2 96.85) (end 140.32 96.85) (width 0.5) (layer B.Cu) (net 12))
 (segment (start 144.415 105.285) (end 144.4 105.27) (width 0.25) (layer B.Cu) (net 3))
 (segment (start 146.125 105.285) (end 144.415 105.285) (width 0.25) (layer B.Cu) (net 3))
 (segment (start 146.125 105.285) (end 147.915 105.285) (width 0.25) (layer B.Cu) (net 3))
 (segment (start 149.185 104.015) (end 151.075 104.015) (width 0.25) (layer B.Cu) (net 3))
 (segment (start 147.915 105.285) (end 149.185 104.015) (width 0.25) (layer B.Cu) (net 3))
 (segment (start 151.1 103.99) (end 151.075 104.015) (width 0.25) (layer B.Cu) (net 3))
 (segment (start 152.9 103.99) (end 151.1 103.99) (width 0.25) (layer B.Cu) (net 3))
 (segment (start 143.62 105.27) (end 143.35 105) (width 0.25) (layer B.Cu) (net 3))
 (segment (start 144.4 105.27) (end 143.52 105.27) (width 0.25) (layer B.Cu) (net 3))
 (segment (start 139.45 105.65) (end 139.4 105.7) (width 0.5) (layer B.Cu) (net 7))
 (segment (start 139.4 102.35) (end 139.45 102.3) (width 0.5) (layer B.Cu) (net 7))
 (segment (start 139.4 105.7) (end 139.4 102.35) (width 0.5) (layer B.Cu) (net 7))
 (segment (start 140.43 106.63) (end 139.7 105.9) (width 0.5) (layer B.Cu) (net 7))
 (segment (start 141.75 106.63) (end 140.43 106.63) (width 0.5) (layer B.Cu) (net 7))
 (segment (start 150.65 94.725) (end 150.65 93.65) (width 0.25) (layer B.Cu) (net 13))
 (segment (start 151.05 93.25) (end 151.75 93.25) (width 0.25) (layer B.Cu) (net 13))
 (segment (start 150.65 93.65) (end 151.05 93.25) (width 0.25) (layer B.Cu) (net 13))
 (segment (start 146.35 99.3) (end 146.6 99.05) (width 0.5) (layer B.Cu) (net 13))
 (segment (start 145.5 99.3) (end 146.35 99.3) (width 0.5) (layer B.Cu) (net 13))
 (segment (start 146.6 99.05) (end 146.6 95.7) (width 0.5) (layer B.Cu) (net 13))
 (segment (start 147.6 95.55) (end 146.75 95.55) (width 0.5) (layer B.Cu) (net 13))
 (segment (start 147.6 95.55) (end 148.425 94.725) (width 0.5) (layer B.Cu) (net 13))
 (segment (start 148.425 94.725) (end 150.65 94.725) (width 0.5) (layer B.Cu) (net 13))
 (segment (start 146.6 95.7) (end 146.75 95.55) (width 0.5) (layer B.Cu) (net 13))
 (segment (start 156.15 100.45) (end 156.2 100.5) (width 0.25) (layer B.Cu) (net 9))
 (segment (start 154.66 100.45) (end 156.15 100.45) (width 0.25) (layer B.Cu) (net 9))
 (segment (start 156.1 99.4) (end 156.2 99.5) (width 0.25) (layer B.Cu) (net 10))
 (segment (start 154.66 99.4) (end 156.1 99.4) (width 0.25) (layer B.Cu) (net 10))
 (segment (start 142.5 94) (end 143.1 93.4) (width 0.5) (layer B.Cu) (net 1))
 (segment (start 141.6 94) (end 142.5 94) (width 0.5) (layer B.Cu) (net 1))
 (segment (start 143.6 93.4) (end 143.1 93.4) (width 0.5) (layer B.Cu) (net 1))
 (segment (start 139.7 94) (end 139.4 94.3) (width 0.5) (layer B.Cu) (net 1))
 (segment (start 141.6 94) (end 139.7 94) (width 0.5) (layer B.Cu) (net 1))
 (segment (start 142.35 100.05) (end 144.3 102) (width 0.5) (layer B.Cu) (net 1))
 (segment (start 144.3 102) (end 144.3 102.69) (width 0.5) (layer B.Cu) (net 1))
 (segment (start 139.25 100.05) (end 142.35 100.05) (width 0.5) (layer B.Cu) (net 1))
 (segment (start 138.875 99.675) (end 139.25 100.05) (width 0.5) (layer B.Cu) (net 1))
 (segment (start 138.875 94.825) (end 138.875 99.675) (width 0.5) (layer B.Cu) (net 1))
 (segment (start 139.4 94.3) (end 138.875 94.825) (width 0.5) (layer B.Cu) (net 1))
 (segment (start 146.125 102.745) (end 144.945 102.745) (width 0.5) (layer B.Cu) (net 1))
 (segment (start 144.89 102.69) (end 144.3 102.69) (width 0.5) (layer B.Cu) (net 1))
 (segment (start 144.945 102.745) (end 144.89 102.69) (width 0.5) (layer B.Cu) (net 1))
 (segment (start 152.9 107.01) (end 152.56 107.01) (width 0.5) (layer B.Cu) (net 1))
 (segment (start 152.105 106.555) (end 151.075 106.555) (width 0.5) (layer B.Cu) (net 1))
 (segment (start 152.56 107.01) (end 152.105 106.555) (width 0.5) (layer B.Cu) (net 1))
 (segment (start 146.125 102.745) (end 148.655 102.745) (width 0.5) (layer B.Cu) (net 1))
 (segment (start 148.655 102.745) (end 149.5 101.9) (width 0.5) (layer B.Cu) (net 1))
 (segment (start 149.5 101.9) (end 152.4 101.9) (width 0.5) (layer B.Cu) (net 1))
 (segment (start 152.4 101.9) (end 154 103.5) (width 0.5) (layer B.Cu) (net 1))
 (segment (start 154 103.5) (end 154 106.55) (width 0.5) (layer B.Cu) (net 1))
 (segment (start 153.54 107.01) (end 152.9 107.01) (width 0.5) (layer B.Cu) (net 1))
 (segment (start 154 106.55) (end 153.54 107.01) (width 0.5) (layer B.Cu) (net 1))
 (segment (start 143.1 102.69) (end 143.1 101.95) (width 0.25) (layer B.Cu) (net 11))
 (segment (start 142.5 101.35) (end 141.45 101.35) (width 0.25) (layer B.Cu) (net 11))
 (segment (start 143.1 101.95) (end 142.5 101.35) (width 0.25) (layer B.Cu) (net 11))
 (segment (start 141.15 101.05) (end 139.1 101.05) (width 0.25) (layer B.Cu) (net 11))
 (segment (start 141.45 101.35) (end 141.15 101.05) (width 0.25) (layer B.Cu) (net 11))
 (segment (start 147.7 100.7) (end 147.5 100.9) (width 0.25) (layer B.Cu) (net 14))
 (segment (start 147.7 99.3) (end 147.7 100.7) (width 0.25) (layer B.Cu) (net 14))
 (segment (start 147.25 100.65) (end 147.5 100.9) (width 0.25) (layer B.Cu) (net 14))
 (segment (start 146.36 100.65) (end 147.25 100.65) (width 0.25) (layer B.Cu) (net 14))
 (segment (start 143.649231 98.562436) (end 143.649231 97.512436) (width 0.25) (layer B.Cu) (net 6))
 (segment (start 143.672436 97.4) (end 143.56 97.512436) (width 0.25) (layer B.Cu) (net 6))
 (segment (start 145.5 97.4) (end 143.672436 97.4) (width 0.25) (layer B.Cu) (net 6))
 (segment (start 144.3 103.71) (end 143.1 103.71) (width 0.25) (layer B.Cu) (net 4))
 (segment (start 144.3 103.71) (end 144.71 103.71) (width 0.25) (layer B.Cu) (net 4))
 (segment (start 145.015 104.015) (end 146.125 104.015) (width 0.25) (layer B.Cu) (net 4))
 (segment (start 144.71 103.71) (end 145.015 104.015) (width 0.25) (layer B.Cu) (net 4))
 (segment (start 143.25 108.2) (end 144.3 108.2) (width 0.25) (layer B.Cu) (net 4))
 (segment (start 142.45 107.4) (end 143.25 108.2) (width 0.25) (layer B.Cu) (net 4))
 (segment (start 142.45 103.95) (end 142.45 107.4) (width 0.25) (layer B.Cu) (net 4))
 (segment (start 142.69 103.71) (end 142.45 103.95) (width 0.25) (layer B.Cu) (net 4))
 (segment (start 143.1 103.71) (end 142.69 103.71) (width 0.25) (layer B.Cu) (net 4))
 (segment (start 152.625 105.285) (end 152.9 105.01) (width 0.25) (layer B.Cu) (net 2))
 (segment (start 151.075 105.285) (end 152.625 105.285) (width 0.25) (layer B.Cu) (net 2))
 (segment (start 152.9 105.56) (end 152.625 105.285) (width 0.25) (layer B.Cu) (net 2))
 (segment (start 152.9 105.99) (end 152.9 105.56) (width 0.25) (layer B.Cu) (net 2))
 (segment (start 151.075 105.285) (end 149.365 105.285) (width 0.25) (layer B.Cu) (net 2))
 (segment (start 148.45 106.2) (end 148.45 107.25) (width 0.25) (layer B.Cu) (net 2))
 (segment (start 149.365 105.285) (end 148.45 106.2) (width 0.25) (layer B.Cu) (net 2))
 (segment (start 147.5 108.2) (end 146.1 108.2) (width 0.25) (layer B.Cu) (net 2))
 (segment (start 148.45 107.25) (end 147.5 108.2) (width 0.25) (layer B.Cu) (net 2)))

